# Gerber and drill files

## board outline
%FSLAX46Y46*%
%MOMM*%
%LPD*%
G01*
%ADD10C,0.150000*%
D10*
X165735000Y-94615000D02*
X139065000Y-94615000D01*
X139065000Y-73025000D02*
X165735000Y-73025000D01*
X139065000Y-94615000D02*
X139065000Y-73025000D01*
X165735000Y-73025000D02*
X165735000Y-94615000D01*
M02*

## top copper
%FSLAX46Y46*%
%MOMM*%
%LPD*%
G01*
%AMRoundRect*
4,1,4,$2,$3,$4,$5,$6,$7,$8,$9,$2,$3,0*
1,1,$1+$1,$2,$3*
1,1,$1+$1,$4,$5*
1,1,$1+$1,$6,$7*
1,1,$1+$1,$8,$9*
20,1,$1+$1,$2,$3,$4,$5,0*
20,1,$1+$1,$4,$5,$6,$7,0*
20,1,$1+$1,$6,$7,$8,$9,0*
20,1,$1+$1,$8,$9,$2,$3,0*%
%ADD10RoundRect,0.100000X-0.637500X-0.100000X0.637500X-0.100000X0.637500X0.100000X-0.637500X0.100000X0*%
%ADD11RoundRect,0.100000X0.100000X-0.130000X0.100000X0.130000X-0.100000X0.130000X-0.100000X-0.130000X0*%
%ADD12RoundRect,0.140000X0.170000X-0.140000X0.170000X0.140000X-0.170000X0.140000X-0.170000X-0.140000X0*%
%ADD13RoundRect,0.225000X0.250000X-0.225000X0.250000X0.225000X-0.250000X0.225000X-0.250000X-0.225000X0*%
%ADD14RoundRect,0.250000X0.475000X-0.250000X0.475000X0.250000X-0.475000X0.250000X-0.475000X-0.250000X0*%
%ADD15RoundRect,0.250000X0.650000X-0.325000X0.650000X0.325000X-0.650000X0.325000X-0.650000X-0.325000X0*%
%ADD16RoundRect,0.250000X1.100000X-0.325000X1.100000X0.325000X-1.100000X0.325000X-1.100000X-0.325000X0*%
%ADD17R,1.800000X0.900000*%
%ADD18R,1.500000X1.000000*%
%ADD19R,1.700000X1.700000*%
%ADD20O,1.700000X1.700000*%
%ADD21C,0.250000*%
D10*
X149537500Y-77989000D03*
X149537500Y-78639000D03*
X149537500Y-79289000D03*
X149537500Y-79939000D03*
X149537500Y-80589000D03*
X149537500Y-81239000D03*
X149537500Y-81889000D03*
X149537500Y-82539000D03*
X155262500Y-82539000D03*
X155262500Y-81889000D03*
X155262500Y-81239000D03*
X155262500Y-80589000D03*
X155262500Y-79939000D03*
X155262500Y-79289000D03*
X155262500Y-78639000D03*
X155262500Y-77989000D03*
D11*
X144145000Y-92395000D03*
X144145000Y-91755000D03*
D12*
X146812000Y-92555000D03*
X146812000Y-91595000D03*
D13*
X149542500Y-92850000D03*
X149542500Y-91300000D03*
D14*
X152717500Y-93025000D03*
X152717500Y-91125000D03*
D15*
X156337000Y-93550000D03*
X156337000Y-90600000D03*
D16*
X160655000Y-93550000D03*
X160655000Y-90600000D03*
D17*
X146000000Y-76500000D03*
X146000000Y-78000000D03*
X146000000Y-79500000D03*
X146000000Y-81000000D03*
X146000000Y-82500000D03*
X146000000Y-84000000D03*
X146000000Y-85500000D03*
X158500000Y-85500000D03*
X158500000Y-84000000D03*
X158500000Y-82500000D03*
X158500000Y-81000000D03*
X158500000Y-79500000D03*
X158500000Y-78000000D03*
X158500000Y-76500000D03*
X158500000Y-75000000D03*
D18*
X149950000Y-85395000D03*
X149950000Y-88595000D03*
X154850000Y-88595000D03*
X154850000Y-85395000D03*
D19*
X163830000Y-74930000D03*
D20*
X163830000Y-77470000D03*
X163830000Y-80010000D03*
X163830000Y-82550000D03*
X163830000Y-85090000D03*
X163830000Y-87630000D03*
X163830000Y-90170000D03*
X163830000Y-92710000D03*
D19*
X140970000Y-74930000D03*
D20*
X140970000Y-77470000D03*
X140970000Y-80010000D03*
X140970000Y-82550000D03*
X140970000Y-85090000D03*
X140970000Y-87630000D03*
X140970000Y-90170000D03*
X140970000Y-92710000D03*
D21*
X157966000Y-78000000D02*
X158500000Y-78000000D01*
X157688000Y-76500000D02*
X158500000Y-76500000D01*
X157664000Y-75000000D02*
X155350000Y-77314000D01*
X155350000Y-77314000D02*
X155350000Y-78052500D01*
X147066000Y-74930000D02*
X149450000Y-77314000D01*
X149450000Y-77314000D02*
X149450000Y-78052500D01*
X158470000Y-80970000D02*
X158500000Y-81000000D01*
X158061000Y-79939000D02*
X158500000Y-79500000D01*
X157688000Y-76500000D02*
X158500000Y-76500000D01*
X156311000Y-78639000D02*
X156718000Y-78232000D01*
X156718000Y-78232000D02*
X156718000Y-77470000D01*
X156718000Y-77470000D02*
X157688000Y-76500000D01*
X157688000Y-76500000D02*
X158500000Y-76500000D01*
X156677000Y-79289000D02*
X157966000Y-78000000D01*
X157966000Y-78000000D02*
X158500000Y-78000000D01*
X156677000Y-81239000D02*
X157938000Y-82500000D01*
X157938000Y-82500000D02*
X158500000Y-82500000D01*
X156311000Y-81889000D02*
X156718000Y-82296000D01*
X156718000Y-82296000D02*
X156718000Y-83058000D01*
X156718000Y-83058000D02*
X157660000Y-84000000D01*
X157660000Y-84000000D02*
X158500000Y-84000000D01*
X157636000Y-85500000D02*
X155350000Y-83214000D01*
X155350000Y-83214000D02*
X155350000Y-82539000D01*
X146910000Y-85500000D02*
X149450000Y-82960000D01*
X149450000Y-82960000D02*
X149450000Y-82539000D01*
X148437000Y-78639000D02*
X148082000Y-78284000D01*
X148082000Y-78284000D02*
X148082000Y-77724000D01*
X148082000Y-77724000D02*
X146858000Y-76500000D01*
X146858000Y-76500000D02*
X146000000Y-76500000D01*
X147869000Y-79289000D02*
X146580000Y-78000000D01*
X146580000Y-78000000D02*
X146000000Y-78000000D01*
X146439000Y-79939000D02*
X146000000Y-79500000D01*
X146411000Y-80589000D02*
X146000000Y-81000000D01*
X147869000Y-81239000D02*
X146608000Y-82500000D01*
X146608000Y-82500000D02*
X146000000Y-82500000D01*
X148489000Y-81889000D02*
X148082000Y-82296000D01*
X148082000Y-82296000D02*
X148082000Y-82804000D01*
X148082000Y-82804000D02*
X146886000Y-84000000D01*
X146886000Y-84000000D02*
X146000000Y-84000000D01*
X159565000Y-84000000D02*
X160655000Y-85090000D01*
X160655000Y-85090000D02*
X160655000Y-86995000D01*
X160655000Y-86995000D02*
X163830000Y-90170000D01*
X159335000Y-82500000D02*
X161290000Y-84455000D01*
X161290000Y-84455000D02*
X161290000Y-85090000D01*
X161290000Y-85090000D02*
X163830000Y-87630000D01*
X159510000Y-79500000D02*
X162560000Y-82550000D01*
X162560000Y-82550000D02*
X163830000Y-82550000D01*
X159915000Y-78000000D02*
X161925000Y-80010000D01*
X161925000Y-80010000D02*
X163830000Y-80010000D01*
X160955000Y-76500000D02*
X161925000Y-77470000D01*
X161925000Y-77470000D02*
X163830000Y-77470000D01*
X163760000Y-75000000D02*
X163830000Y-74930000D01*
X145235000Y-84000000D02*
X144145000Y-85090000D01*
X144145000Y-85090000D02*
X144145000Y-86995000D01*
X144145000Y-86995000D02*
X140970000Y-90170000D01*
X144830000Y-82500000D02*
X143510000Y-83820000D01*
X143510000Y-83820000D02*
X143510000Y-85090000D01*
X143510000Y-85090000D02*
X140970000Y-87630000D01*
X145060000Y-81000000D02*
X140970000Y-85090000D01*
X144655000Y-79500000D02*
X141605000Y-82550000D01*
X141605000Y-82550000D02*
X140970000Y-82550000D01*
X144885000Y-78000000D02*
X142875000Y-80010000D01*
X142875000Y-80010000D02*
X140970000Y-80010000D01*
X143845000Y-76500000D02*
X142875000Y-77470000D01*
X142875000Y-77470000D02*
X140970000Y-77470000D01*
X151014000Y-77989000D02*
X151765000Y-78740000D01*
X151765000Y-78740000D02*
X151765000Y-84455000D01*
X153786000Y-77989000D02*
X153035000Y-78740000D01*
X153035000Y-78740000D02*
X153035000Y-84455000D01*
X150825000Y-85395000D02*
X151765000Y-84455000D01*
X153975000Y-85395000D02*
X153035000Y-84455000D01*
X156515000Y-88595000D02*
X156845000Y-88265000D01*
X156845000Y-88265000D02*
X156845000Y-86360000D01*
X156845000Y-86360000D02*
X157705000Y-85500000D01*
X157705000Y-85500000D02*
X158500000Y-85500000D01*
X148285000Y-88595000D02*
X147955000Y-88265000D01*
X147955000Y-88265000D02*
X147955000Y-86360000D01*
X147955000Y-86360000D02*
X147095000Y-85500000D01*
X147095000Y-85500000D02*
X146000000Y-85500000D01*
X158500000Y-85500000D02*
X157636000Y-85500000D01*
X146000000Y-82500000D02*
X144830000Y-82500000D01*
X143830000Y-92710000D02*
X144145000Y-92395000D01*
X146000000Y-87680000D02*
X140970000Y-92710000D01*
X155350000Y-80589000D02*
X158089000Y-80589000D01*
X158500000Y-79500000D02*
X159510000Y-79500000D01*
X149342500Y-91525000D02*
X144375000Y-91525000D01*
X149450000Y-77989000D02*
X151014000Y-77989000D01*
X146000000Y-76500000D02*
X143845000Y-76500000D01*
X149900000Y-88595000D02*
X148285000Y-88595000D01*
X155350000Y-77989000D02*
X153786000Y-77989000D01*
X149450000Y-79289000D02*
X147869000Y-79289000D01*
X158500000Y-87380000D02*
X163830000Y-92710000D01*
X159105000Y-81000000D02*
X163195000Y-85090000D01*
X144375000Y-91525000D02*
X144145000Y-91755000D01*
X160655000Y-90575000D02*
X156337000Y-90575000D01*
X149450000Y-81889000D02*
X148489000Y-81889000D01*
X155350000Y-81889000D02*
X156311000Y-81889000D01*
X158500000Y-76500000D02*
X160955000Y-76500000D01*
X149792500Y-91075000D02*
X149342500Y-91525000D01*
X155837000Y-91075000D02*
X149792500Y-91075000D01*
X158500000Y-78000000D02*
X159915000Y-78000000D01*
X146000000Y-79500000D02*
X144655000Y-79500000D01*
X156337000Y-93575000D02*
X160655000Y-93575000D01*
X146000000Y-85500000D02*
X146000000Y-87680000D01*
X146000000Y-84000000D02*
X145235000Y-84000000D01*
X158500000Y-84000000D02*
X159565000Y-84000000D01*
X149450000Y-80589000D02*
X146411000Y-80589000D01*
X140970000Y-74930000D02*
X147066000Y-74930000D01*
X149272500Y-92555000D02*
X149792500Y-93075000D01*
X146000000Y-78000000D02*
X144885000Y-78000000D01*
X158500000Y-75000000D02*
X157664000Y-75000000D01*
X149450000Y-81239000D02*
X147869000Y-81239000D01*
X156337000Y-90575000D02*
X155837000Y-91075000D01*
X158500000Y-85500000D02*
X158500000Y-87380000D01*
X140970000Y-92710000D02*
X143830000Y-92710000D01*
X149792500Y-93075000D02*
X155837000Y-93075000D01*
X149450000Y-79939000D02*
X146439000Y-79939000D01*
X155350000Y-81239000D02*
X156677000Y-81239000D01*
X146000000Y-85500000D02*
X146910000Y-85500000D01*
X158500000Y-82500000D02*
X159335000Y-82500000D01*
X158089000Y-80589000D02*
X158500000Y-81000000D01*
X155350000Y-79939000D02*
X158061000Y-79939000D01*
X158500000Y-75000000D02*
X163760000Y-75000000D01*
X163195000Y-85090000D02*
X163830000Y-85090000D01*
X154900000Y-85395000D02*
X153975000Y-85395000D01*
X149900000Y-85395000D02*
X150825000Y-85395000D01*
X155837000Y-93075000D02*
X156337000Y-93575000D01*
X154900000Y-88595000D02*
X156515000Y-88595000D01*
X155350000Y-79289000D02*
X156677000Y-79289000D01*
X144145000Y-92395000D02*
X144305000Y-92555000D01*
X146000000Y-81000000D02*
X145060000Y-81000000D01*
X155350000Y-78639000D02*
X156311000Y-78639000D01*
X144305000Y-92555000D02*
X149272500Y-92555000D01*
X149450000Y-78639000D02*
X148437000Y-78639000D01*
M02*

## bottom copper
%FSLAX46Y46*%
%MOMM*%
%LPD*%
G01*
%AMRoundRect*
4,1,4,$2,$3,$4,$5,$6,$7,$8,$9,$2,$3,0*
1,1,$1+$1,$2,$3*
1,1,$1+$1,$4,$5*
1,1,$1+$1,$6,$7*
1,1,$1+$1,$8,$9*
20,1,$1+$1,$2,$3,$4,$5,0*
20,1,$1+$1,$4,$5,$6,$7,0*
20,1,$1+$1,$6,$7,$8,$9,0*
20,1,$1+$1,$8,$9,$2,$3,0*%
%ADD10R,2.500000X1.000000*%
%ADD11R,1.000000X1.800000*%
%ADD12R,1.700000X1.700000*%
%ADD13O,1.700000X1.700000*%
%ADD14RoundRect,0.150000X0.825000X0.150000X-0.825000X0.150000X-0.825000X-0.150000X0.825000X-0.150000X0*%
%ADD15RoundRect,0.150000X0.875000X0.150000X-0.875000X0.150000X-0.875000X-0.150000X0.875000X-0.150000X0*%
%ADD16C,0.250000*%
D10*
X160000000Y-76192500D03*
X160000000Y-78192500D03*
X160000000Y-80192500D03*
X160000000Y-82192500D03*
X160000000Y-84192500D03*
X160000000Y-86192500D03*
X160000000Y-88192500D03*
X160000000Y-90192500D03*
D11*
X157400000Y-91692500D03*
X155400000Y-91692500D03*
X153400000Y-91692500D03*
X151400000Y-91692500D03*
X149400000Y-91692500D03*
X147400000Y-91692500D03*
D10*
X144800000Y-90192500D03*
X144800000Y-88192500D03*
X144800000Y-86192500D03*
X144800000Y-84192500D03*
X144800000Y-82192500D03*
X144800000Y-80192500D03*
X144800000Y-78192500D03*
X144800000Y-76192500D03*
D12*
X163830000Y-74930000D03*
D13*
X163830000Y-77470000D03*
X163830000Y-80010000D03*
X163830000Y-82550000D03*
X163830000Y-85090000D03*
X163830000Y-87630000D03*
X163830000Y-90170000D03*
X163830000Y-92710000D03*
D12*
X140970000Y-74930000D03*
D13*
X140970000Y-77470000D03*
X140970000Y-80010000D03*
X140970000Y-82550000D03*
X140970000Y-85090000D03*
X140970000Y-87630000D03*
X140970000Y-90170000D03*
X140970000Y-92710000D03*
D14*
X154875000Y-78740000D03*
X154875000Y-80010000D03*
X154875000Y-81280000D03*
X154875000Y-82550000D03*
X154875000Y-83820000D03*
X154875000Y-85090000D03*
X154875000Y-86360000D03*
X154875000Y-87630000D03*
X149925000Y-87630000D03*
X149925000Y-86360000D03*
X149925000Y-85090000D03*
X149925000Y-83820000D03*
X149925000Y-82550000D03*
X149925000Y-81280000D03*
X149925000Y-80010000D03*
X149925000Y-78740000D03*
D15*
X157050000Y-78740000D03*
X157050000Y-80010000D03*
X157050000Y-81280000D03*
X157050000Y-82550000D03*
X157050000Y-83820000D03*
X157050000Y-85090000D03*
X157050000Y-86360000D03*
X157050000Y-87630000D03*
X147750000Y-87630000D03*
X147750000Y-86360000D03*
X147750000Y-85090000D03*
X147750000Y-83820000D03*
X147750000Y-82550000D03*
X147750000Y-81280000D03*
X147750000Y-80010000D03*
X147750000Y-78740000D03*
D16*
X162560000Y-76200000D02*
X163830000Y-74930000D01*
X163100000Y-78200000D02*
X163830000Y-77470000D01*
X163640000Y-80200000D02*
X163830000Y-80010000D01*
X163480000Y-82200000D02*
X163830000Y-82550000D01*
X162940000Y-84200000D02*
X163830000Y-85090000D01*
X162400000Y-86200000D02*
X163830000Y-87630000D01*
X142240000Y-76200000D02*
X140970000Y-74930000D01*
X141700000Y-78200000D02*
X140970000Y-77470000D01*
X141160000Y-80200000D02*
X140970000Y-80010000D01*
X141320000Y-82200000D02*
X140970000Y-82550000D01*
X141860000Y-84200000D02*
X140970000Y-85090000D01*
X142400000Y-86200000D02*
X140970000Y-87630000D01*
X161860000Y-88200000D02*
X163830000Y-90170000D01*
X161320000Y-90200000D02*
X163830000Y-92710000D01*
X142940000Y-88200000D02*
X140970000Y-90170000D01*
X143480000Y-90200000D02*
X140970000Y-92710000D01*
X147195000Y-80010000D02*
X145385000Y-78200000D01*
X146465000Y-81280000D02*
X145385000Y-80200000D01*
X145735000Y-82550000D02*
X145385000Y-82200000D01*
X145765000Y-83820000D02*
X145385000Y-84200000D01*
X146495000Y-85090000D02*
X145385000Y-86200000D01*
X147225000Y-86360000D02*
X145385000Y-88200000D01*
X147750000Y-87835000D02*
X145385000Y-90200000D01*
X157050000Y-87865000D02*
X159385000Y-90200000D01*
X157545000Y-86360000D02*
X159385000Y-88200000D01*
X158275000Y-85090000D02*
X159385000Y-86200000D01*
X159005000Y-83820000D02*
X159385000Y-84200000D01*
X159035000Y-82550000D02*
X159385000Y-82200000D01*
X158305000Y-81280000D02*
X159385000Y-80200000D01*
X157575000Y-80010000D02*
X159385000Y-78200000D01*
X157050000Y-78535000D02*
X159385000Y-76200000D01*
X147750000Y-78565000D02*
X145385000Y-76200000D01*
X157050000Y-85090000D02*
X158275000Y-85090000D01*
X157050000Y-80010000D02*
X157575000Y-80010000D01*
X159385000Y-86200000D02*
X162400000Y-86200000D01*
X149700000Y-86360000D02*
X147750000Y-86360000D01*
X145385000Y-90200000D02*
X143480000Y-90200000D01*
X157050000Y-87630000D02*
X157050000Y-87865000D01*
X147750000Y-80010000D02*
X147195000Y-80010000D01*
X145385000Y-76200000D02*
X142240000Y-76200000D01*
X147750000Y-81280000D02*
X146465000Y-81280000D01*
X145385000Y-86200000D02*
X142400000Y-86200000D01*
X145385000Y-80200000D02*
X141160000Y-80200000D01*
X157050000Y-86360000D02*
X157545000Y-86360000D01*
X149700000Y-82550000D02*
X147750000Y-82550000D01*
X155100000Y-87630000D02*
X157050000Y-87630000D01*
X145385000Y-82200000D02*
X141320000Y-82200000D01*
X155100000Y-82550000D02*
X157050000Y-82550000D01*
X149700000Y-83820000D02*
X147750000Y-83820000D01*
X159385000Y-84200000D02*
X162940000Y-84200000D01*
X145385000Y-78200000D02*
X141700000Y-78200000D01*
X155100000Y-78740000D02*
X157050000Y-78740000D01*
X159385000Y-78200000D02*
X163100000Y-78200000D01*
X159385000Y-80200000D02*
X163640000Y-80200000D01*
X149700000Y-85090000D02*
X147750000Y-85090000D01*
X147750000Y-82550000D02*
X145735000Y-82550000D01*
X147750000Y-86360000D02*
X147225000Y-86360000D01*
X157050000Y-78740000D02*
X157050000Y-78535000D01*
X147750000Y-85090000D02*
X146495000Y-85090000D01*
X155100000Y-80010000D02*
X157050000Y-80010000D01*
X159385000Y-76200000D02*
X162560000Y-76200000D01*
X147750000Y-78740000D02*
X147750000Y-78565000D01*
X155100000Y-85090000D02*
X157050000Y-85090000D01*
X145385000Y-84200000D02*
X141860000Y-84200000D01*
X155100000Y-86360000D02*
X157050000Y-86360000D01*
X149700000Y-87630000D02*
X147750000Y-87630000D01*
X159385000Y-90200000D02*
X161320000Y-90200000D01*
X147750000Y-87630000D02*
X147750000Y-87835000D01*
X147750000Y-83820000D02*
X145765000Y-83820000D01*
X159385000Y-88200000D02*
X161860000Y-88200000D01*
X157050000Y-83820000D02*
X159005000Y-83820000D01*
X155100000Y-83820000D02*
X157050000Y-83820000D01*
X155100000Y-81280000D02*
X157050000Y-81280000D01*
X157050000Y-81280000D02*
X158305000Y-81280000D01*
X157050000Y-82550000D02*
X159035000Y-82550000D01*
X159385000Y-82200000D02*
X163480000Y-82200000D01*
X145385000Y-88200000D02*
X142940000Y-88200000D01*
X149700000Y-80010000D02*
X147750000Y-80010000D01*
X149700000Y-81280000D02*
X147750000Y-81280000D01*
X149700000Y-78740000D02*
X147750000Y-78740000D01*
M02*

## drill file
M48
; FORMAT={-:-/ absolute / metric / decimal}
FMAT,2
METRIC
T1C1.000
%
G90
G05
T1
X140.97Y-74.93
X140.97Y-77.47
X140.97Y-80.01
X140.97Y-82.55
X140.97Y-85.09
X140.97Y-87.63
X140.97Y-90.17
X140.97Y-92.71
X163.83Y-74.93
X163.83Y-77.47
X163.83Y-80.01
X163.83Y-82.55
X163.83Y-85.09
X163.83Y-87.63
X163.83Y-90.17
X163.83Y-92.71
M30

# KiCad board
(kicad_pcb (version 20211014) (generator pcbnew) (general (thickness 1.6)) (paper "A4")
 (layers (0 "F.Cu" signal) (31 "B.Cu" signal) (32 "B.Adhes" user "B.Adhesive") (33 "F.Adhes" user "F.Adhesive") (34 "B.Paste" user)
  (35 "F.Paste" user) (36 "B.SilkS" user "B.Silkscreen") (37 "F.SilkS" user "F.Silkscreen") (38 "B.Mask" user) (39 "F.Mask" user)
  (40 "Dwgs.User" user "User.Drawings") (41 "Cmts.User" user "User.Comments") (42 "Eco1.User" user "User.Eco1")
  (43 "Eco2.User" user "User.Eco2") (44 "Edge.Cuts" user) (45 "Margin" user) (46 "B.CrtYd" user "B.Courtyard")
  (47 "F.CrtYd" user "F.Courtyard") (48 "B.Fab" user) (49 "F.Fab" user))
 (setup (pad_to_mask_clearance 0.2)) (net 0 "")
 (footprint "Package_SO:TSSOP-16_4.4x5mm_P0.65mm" (layer "F.Cu") (at 152.4 80.264)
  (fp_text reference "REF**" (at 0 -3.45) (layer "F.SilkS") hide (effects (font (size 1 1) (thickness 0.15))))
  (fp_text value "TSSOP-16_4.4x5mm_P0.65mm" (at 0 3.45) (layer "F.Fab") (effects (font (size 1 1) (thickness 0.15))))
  (pad "1" smd roundrect (at -2.8625 -2.275) (size 1.475 0.4) (layers "F.Cu" "F.Paste" "F.Mask") (roundrect_rratio 0.25))
  (pad "2" smd roundrect (at -2.8625 -1.625) (size 1.475 0.4) (layers "F.Cu" "F.Paste" "F.Mask") (roundrect_rratio 0.25))
  (pad "3" smd roundrect (at -2.8625 -0.975) (size 1.475 0.4) (layers "F.Cu" "F.Paste" "F.Mask") (roundrect_rratio 0.25))
  (pad "4" smd roundrect (at -2.8625 -0.325) (size 1.475 0.4) (layers "F.Cu" "F.Paste" "F.Mask") (roundrect_rratio 0.25))
  (pad "5" smd roundrect (at -2.8625 0.325) (size 1.475 0.4) (layers "F.Cu" "F.Paste" "F.Mask") (roundrect_rratio 0.25))
  (pad "6" smd roundrect (at -2.8625 0.975) (size 1.475 0.4) (layers "F.Cu" "F.Paste" "F.Mask") (roundrect_rratio 0.25))
  (pad "7" smd roundrect (at -2.8625 1.625) (size 1.475 0.4) (layers "F.Cu" "F.Paste" "F.Mask") (roundrect_rratio 0.25))
  (pad "8" smd roundrect (at -2.8625 2.275) (size 1.475 0.4) (layers "F.Cu" "F.Paste" "F.Mask") (roundrect_rratio 0.25))
  (pad "9" smd roundrect (at 2.8625 2.275) (size 1.475 0.4) (layers "F.Cu" "F.Paste" "F.Mask") (roundrect_rratio 0.25))
  (pad "10" smd roundrect (at 2.8625 1.625) (size 1.475 0.4) (layers "F.Cu" "F.Paste" "F.Mask") (roundrect_rratio 0.25))
  (pad "11" smd roundrect (at 2.8625 0.975) (size 1.475 0.4) (layers "F.Cu" "F.Paste" "F.Mask") (roundrect_rratio 0.25))
  (pad "12" smd roundrect (at 2.8625 0.325) (size 1.475 0.4) (layers "F.Cu" "F.Paste" "F.Mask") (roundrect_rratio 0.25))
  (pad "13" smd roundrect (at 2.8625 -0.325) (size 1.475 0.4) (layers "F.Cu" "F.Paste" "F.Mask") (roundrect_rratio 0.25))
  (pad "14" smd roundrect (at 2.8625 -0.975) (size 1.475 0.4) (layers "F.Cu" "F.Paste" "F.Mask") (roundrect_rratio 0.25))
  (pad "15" smd roundrect (at 2.8625 -1.625) (size 1.475 0.4) (layers "F.Cu" "F.Paste" "F.Mask") (roundrect_rratio 0.25))
  (pad "16" smd roundrect (at 2.8625 -2.275) (size 1.475 0.4) (layers "F.Cu" "F.Paste" "F.Mask") (roundrect_rratio 0.25)))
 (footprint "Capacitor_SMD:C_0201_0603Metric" (layer "F.Cu") (at 144.145 92.075 90)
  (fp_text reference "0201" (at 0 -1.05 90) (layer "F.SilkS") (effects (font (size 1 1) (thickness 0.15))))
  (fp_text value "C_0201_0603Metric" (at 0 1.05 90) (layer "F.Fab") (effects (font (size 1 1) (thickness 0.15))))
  (pad "" smd roundrect (at -0.345 0 90) (size 0.318 0.36) (layers "F.Paste") (roundrect_rratio 0.25))
  (pad "" smd roundrect (at 0.345 0 90) (size 0.318 0.36) (layers "F.Paste") (roundrect_rratio 0.25))
  (pad "1" smd roundrect (at -0.32 0 90) (size 0.46 0.4) (layers "F.Cu" "F.Mask") (roundrect_rratio 0.25))
  (pad "2" smd roundrect (at 0.32 0 90) (size 0.46 0.4) (layers "F.Cu" "F.Mask") (roundrect_rratio 0.25)))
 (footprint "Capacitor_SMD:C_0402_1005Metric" (layer "F.Cu") (at 146.812 92.075 90)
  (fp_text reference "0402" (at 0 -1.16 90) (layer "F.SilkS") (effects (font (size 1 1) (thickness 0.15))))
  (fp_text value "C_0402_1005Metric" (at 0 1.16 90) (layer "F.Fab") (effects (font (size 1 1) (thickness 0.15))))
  (pad "1" smd roundrect (at -0.48 0 90) (size 0.56 0.62) (layers "F.Cu" "F.Paste" "F.Mask") (roundrect_rratio 0.25))
  (pad "2" smd roundrect (at 0.48 0 90) (size 0.56 0.62) (layers "F.Cu" "F.Paste" "F.Mask") (roundrect_rratio 0.25)))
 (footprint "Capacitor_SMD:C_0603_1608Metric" (layer "F.Cu") (at 149.5425 92.075 90)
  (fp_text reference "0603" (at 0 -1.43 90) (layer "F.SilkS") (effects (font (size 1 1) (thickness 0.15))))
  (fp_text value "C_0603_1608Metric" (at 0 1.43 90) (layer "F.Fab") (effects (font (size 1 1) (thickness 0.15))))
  (pad "1" smd roundrect (at -0.775 0 90) (size 0.9 0.95) (layers "F.Cu" "F.Paste" "F.Mask") (roundrect_rratio 0.25))
  (pad "2" smd roundrect (at 0.775 0 90) (size 0.9 0.95) (layers "F.Cu" "F.Paste" "F.Mask") (roundrect_rratio 0.25)))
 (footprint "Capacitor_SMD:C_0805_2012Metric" (layer "F.Cu") (at 152.7175 92.075 90)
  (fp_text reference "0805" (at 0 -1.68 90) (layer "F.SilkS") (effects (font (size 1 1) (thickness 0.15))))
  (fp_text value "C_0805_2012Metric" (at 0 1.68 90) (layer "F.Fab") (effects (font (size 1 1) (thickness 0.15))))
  (pad "1" smd roundrect (at -0.95 0 90) (size 1 1.45) (layers "F.Cu" "F.Paste" "F.Mask") (roundrect_rratio 0.25))
  (pad "2" smd roundrect (at 0.95 0 90) (size 1 1.45) (layers "F.Cu" "F.Paste" "F.Mask") (roundrect_rratio 0.25)))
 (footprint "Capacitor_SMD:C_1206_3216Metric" (layer "F.Cu") (at 156.337 92.075 90)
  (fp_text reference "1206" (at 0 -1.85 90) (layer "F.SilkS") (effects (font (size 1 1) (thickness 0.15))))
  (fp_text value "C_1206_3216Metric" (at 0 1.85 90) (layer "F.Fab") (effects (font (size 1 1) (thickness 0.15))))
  (pad "1" smd roundrect (at -1.475 0 90) (size 1.15 1.8) (layers "F.Cu" "F.Paste" "F.Mask") (roundrect_rratio 0.217391))
  (pad "2" smd roundrect (at 1.475 0 90) (size 1.15 1.8) (layers "F.Cu" "F.Paste" "F.Mask") (roundrect_rratio 0.217391)))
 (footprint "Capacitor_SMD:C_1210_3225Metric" (layer "F.Cu") (at 160.655 92.075 90)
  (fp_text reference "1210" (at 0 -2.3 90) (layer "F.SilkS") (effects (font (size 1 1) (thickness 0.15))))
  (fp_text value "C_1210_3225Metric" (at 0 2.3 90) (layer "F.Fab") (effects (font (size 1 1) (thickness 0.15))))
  (pad "1" smd roundrect (at -1.475 0 90) (size 1.15 2.7) (layers "F.Cu" "F.Paste" "F.Mask") (roundrect_rratio 0.217391))
  (pad "2" smd roundrect (at 1.475 0 90) (size 1.15 2.7) (layers "F.Cu" "F.Paste" "F.Mask") (roundrect_rratio 0.217391)))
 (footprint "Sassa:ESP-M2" (layer "F.Cu") (at 146 76.5)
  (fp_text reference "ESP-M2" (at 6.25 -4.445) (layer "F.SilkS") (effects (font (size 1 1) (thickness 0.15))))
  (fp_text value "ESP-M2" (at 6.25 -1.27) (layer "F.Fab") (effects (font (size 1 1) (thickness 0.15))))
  (pad "1" smd rect (at 0 0) (size 1.8 0.9) (layers "F.Cu" "F.Paste" "F.Mask"))
  (pad "2" smd rect (at 0 1.5) (size 1.8 0.9) (layers "F.Cu" "F.Paste" "F.Mask"))
  (pad "3" smd rect (at 0 3) (size 1.8 0.9) (layers "F.Cu" "F.Paste" "F.Mask"))
  (pad "4" smd rect (at 0 4.5) (size 1.8 0.9) (layers "F.Cu" "F.Paste" "F.Mask"))
  (pad "5" smd rect (at 0 6) (size 1.8 0.9) (layers "F.Cu" "F.Paste" "F.Mask"))
  (pad "6" smd rect (at 0 7.5) (size 1.8 0.9) (layers "F.Cu" "F.Paste" "F.Mask"))
  (pad "7" smd rect (at 0 9) (size 1.8 0.9) (layers "F.Cu" "F.Paste" "F.Mask"))
  (pad "8" smd rect (at 12.5 9) (size 1.8 0.9) (layers "F.Cu" "F.Paste" "F.Mask"))
  (pad "9" smd rect (at 12.5 7.5) (size 1.8 0.9) (layers "F.Cu" "F.Paste" "F.Mask"))
  (pad "10" smd rect (at 12.5 6) (size 1.8 0.9) (layers "F.Cu" "F.Paste" "F.Mask"))
  (pad "11" smd rect (at 12.5 4.5) (size 1.8 0.9) (layers "F.Cu" "F.Paste" "F.Mask"))
  (pad "12" smd rect (at 12.5 3) (size 1.8 0.9) (layers "F.Cu" "F.Paste" "F.Mask"))
  (pad "13" smd rect (at 12.5 1.5) (size 1.8 0.9) (layers "F.Cu" "F.Paste" "F.Mask"))
  (pad "14" smd rect (at 12.5 0) (size 1.8 0.9) (layers "F.Cu" "F.Paste" "F.Mask"))
  (pad "15" smd rect (at 12.5 -1.5) (size 1.8 0.9) (layers "F.Cu" "F.Paste" "F.Mask")))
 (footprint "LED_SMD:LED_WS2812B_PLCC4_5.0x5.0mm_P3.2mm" (layer "F.Cu") (at 152.4 86.995)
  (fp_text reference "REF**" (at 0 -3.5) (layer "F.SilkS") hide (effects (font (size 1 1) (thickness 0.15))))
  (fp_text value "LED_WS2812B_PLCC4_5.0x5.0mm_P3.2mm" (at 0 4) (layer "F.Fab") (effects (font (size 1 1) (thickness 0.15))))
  (pad "1" smd rect (at -2.45 -1.6) (size 1.5 1) (layers "F.Cu" "F.Paste" "F.Mask"))
  (pad "2" smd rect (at -2.45 1.6) (size 1.5 1) (layers "F.Cu" "F.Paste" "F.Mask"))
  (pad "3" smd rect (at 2.45 1.6) (size 1.5 1) (layers "F.Cu" "F.Paste" "F.Mask"))
  (pad "4" smd rect (at 2.45 -1.6) (size 1.5 1) (layers "F.Cu" "F.Paste" "F.Mask")))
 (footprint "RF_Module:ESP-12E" (layer "B.Cu") (at 152.4 79.6925 180)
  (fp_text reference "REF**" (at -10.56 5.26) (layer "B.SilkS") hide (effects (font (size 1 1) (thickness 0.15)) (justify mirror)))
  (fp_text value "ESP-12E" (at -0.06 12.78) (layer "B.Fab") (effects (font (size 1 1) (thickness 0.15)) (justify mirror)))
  (pad "1" smd rect (at -7.6 3.5 180) (size 2.5 1) (layers "B.Cu" "B.Paste" "B.Mask"))
  (pad "2" smd rect (at -7.6 1.5 180) (size 2.5 1) (layers "B.Cu" "B.Paste" "B.Mask"))
  (pad "3" smd rect (at -7.6 -0.5 180) (size 2.5 1) (layers "B.Cu" "B.Paste" "B.Mask"))
  (pad "4" smd rect (at -7.6 -2.5 180) (size 2.5 1) (layers "B.Cu" "B.Paste" "B.Mask"))
  (pad "5" smd rect (at -7.6 -4.5 180) (size 2.5 1) (layers "B.Cu" "B.Paste" "B.Mask"))
  (pad "6" smd rect (at -7.6 -6.5 180) (size 2.5 1) (layers "B.Cu" "B.Paste" "B.Mask"))
  (pad "7" smd rect (at -7.6 -8.5 180) (size 2.5 1) (layers "B.Cu" "B.Paste" "B.Mask"))
  (pad "8" smd rect (at -7.6 -10.5 180) (size 2.5 1) (layers "B.Cu" "B.Paste" "B.Mask"))
  (pad "9" smd rect (at -5 -12 180) (size 1 1.8) (layers "B.Cu" "B.Paste" "B.Mask"))
  (pad "10" smd rect (at -3 -12 180) (size 1 1.8) (layers "B.Cu" "B.Paste" "B.Mask"))
  (pad "11" smd rect (at -1 -12 180) (size 1 1.8) (layers "B.Cu" "B.Paste" "B.Mask"))
  (pad "12" smd rect (at 1 -12 180) (size 1 1.8) (layers "B.Cu" "B.Paste" "B.Mask"))
  (pad "13" smd rect (at 3 -12 180) (size 1 1.8) (layers "B.Cu" "B.Paste" "B.Mask"))
  (pad "14" smd rect (at 5 -12 180) (size 1 1.8) (layers "B.Cu" "B.Paste" "B.Mask"))
  (pad "15" smd rect (at 7.6 -10.5 180) (size 2.5 1) (layers "B.Cu" "B.Paste" "B.Mask"))
  (pad "16" smd rect (at 7.6 -8.5 180) (size 2.5 1) (layers "B.Cu" "B.Paste" "B.Mask"))
  (pad "17" smd rect (at 7.6 -6.5 180) (size 2.5 1) (layers "B.Cu" "B.Paste" "B.Mask"))
  (pad "18" smd rect (at 7.6 -4.5 180) (size 2.5 1) (layers "B.Cu" "B.Paste" "B.Mask"))
  (pad "19" smd rect (at 7.6 -2.5 180) (size 2.5 1) (layers "B.Cu" "B.Paste" "B.Mask"))
  (pad "20" smd rect (at 7.6 -0.5 180) (size 2.5 1) (layers "B.Cu" "B.Paste" "B.Mask"))
  (pad "21" smd rect (at 7.6 1.5 180) (size 2.5 1) (layers "B.Cu" "B.Paste" "B.Mask"))
  (pad "22" smd rect (at 7.6 3.5 180) (size 2.5 1) (layers "B.Cu" "B.Paste" "B.Mask"))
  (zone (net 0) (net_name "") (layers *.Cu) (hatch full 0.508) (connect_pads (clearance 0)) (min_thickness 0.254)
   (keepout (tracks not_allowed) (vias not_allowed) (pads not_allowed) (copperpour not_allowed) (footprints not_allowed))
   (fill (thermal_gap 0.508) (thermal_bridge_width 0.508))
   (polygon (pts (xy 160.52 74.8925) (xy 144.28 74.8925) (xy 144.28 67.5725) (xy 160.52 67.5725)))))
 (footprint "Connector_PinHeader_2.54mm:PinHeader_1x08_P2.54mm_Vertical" (layer "B.Cu") (at 163.83 74.93 180)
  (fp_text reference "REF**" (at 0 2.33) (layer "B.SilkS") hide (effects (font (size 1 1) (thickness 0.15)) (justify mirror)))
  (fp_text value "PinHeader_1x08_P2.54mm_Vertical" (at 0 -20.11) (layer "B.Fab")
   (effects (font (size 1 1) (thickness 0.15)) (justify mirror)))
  (pad "1" thru_hole rect (at 0 0 180) (size 1.7 1.7) (drill 1) (layers *.Cu *.Mask))
  (pad "2" thru_hole oval (at 0 -2.54 180) (size 1.7 1.7) (drill 1) (layers *.Cu *.Mask))
  (pad "3" thru_hole oval (at 0 -5.08 180) (size 1.7 1.7) (drill 1) (layers *.Cu *.Mask))
  (pad "4" thru_hole oval (at 0 -7.62 180) (size 1.7 1.7) (drill 1) (layers *.Cu *.Mask))
  (pad "5" thru_hole oval (at 0 -10.16 180) (size 1.7 1.7) (drill 1) (layers *.Cu *.Mask))
  (pad "6" thru_hole oval (at 0 -12.7 180) (size 1.7 1.7) (drill 1) (layers *.Cu *.Mask))
  (pad "7" thru_hole oval (at 0 -15.24 180) (size 1.7 1.7) (drill 1) (layers *.Cu *.Mask))
  (pad "8" thru_hole oval (at 0 -17.78 180) (size 1.7 1.7) (drill 1) (layers *.Cu *.Mask)))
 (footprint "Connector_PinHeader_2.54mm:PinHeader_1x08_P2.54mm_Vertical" (layer "B.Cu") (at 140.97 74.93 180)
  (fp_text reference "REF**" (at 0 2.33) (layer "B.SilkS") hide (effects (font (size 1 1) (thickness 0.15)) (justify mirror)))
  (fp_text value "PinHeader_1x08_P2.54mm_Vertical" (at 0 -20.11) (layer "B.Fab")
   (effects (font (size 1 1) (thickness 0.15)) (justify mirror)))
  (pad "1" thru_hole rect (at 0 0 180) (size 1.7 1.7) (drill 1) (layers *.Cu *.Mask))
  (pad "2" thru_hole oval (at 0 -2.54 180) (size 1.7 1.7) (drill 1) (layers *.Cu *.Mask))
  (pad "3" thru_hole oval (at 0 -5.08 180) (size 1.7 1.7) (drill 1) (layers *.Cu *.Mask))
  (pad "4" thru_hole oval (at 0 -7.62 180) (size 1.7 1.7) (drill 1) (layers *.Cu *.Mask))
  (pad "5" thru_hole oval (at 0 -10.16 180) (size 1.7 1.7) (drill 1) (layers *.Cu *.Mask))
  (pad "6" thru_hole oval (at 0 -12.7 180) (size 1.7 1.7) (drill 1) (layers *.Cu *.Mask))
  (pad "7" thru_hole oval (at 0 -15.24 180) (size 1.7 1.7) (drill 1) (layers *.Cu *.Mask))
  (pad "8" thru_hole oval (at 0 -17.78 180) (size 1.7 1.7) (drill 1) (layers *.Cu *.Mask)))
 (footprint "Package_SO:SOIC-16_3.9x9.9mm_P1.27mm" (layer "B.Cu") (at 152.4 83.185 180)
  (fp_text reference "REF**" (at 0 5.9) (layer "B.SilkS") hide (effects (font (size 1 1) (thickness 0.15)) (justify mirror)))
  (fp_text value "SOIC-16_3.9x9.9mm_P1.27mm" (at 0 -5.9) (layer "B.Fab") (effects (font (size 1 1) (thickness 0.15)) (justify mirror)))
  (pad "1" smd roundrect (at -2.475 4.445 180) (size 1.95 0.6) (layers "B.Cu" "B.Paste" "B.Mask") (roundrect_rratio 0.25))
  (pad "2" smd roundrect (at -2.475 3.175 180) (size 1.95 0.6) (layers "B.Cu" "B.Paste" "B.Mask") (roundrect_rratio 0.25))
  (pad "3" smd roundrect (at -2.475 1.905 180) (size 1.95 0.6) (layers "B.Cu" "B.Paste" "B.Mask") (roundrect_rratio 0.25))
  (pad "4" smd roundrect (at -2.475 0.635 180) (size 1.95 0.6) (layers "B.Cu" "B.Paste" "B.Mask") (roundrect_rratio 0.25))
  (pad "5" smd roundrect (at -2.475 -0.635 180) (size 1.95 0.6) (layers "B.Cu" "B.Paste" "B.Mask") (roundrect_rratio 0.25))
  (pad "6" smd roundrect (at -2.475 -1.905 180) (size 1.95 0.6) (layers "B.Cu" "B.Paste" "B.Mask") (roundrect_rratio 0.25))
  (pad "7" smd roundrect (at -2.475 -3.175 180) (size 1.95 0.6) (layers "B.Cu" "B.Paste" "B.Mask") (roundrect_rratio 0.25))
  (pad "8" smd roundrect (at -2.475 -4.445 180) (size 1.95 0.6) (layers "B.Cu" "B.Paste" "B.Mask") (roundrect_rratio 0.25))
  (pad "9" smd roundrect (at 2.475 -4.445 180) (size 1.95 0.6) (layers "B.Cu" "B.Paste" "B.Mask") (roundrect_rratio 0.25))
  (pad "10" smd roundrect (at 2.475 -3.175 180) (size 1.95 0.6) (layers "B.Cu" "B.Paste" "B.Mask") (roundrect_rratio 0.25))
  (pad "11" smd roundrect (at 2.475 -1.905 180) (size 1.95 0.6) (layers "B.Cu" "B.Paste" "B.Mask") (roundrect_rratio 0.25))
  (pad "12" smd roundrect (at 2.475 -0.635 180) (size 1.95 0.6) (layers "B.Cu" "B.Paste" "B.Mask") (roundrect_rratio 0.25))
  (pad "13" smd roundrect (at 2.475 0.635 180) (size 1.95 0.6) (layers "B.Cu" "B.Paste" "B.Mask") (roundrect_rratio 0.25))
  (pad "14" smd roundrect (at 2.475 1.905 180) (size 1.95 0.6) (layers "B.Cu" "B.Paste" "B.Mask") (roundrect_rratio 0.25))
  (pad "15" smd roundrect (at 2.475 3.175 180) (size 1.95 0.6) (layers "B.Cu" "B.Paste" "B.Mask") (roundrect_rratio 0.25))
  (pad "16" smd roundrect (at 2.475 4.445 180) (size 1.95 0.6) (layers "B.Cu" "B.Paste" "B.Mask") (roundrect_rratio 0.25)))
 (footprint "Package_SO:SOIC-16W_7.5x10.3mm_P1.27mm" (layer "B.Cu") (at 152.4 83.185 180)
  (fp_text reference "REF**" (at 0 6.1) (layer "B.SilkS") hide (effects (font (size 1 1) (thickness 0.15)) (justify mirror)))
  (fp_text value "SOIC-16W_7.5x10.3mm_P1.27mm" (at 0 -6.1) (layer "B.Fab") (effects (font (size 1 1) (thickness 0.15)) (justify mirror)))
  (pad "1" smd roundrect (at -4.65 4.445 180) (size 2.05 0.6) (layers "B.Cu" "B.Paste" "B.Mask") (roundrect_rratio 0.25))
  (pad "2" smd roundrect (at -4.65 3.175 180) (size 2.05 0.6) (layers "B.Cu" "B.Paste" "B.Mask") (roundrect_rratio 0.25))
  (pad "3" smd roundrect (at -4.65 1.905 180) (size 2.05 0.6) (layers "B.Cu" "B.Paste" "B.Mask") (roundrect_rratio 0.25))
  (pad "4" smd roundrect (at -4.65 0.635 180) (size 2.05 0.6) (layers "B.Cu" "B.Paste" "B.Mask") (roundrect_rratio 0.25))
  (pad "5" smd roundrect (at -4.65 -0.635 180) (size 2.05 0.6) (layers "B.Cu" "B.Paste" "B.Mask") (roundrect_rratio 0.25))
  (pad "6" smd roundrect (at -4.65 -1.905 180) (size 2.05 0.6) (layers "B.Cu" "B.Paste" "B.Mask") (roundrect_rratio 0.25))
  (pad "7" smd roundrect (at -4.65 -3.175 180) (size 2.05 0.6) (layers "B.Cu" "B.Paste" "B.Mask") (roundrect_rratio 0.25))
  (pad "8" smd roundrect (at -4.65 -4.445 180) (size 2.05 0.6) (layers "B.Cu" "B.Paste" "B.Mask") (roundrect_rratio 0.25))
  (pad "9" smd roundrect (at 4.65 -4.445 180) (size 2.05 0.6) (layers "B.Cu" "B.Paste" "B.Mask") (roundrect_rratio 0.25))
  (pad "10" smd roundrect (at 4.65 -3.175 180) (size 2.05 0.6) (layers "B.Cu" "B.Paste" "B.Mask") (roundrect_rratio 0.25))
  (pad "11" smd roundrect (at 4.65 -1.905 180) (size 2.05 0.6) (layers "B.Cu" "B.Paste" "B.Mask") (roundrect_rratio 0.25))
  (pad "12" smd roundrect (at 4.65 -0.635 180) (size 2.05 0.6) (layers "B.Cu" "B.Paste" "B.Mask") (roundrect_rratio 0.25))
  (pad "13" smd roundrect (at 4.65 0.635 180) (size 2.05 0.6) (layers "B.Cu" "B.Paste" "B.Mask") (roundrect_rratio 0.25))
  (pad "14" smd roundrect (at 4.65 1.905 180) (size 2.05 0.6) (layers "B.Cu" "B.Paste" "B.Mask") (roundrect_rratio 0.25))
  (pad "15" smd roundrect (at 4.65 3.175 180) (size 2.05 0.6) (layers "B.Cu" "B.Paste" "B.Mask") (roundrect_rratio 0.25))
  (pad "16" smd roundrect (at 4.65 4.445 180) (size 2.05 0.6) (layers "B.Cu" "B.Paste" "B.Mask") (roundrect_rratio 0.25)))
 (gr_line (start 165.735 94.615) (end 139.065 94.615) (layer "Edge.Cuts") (width 0.15))
 (gr_line (start 139.065 73.025) (end 165.735 73.025) (layer "Edge.Cuts") (width 0.15))
 (gr_line (start 139.065 94.615) (end 139.065 73.025) (layer "Edge.Cuts") (width 0.15))
 (gr_line (start 165.735 73.025) (end 165.735 94.615) (layer "Edge.Cuts") (width 0.15))
 (segment (start 157.966 78) (end 158.5 78) (width 0.25) (layer "F.Cu") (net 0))
 (segment (start 157.688 76.5) (end 158.5 76.5) (width 0.25) (layer "F.Cu") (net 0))
 (segment (start 157.664 75) (end 155.35 77.314) (width 0.25) (layer "F.Cu") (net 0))
 (segment (start 155.35 77.314) (end 155.35 78.0525) (width 0.25) (layer "F.Cu") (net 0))
 (segment (start 147.066 74.93) (end 149.45 77.314) (width 0.25) (layer "F.Cu") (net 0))
 (segment (start 149.45 77.314) (end 149.45 78.0525) (width 0.25) (layer "F.Cu") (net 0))
 (segment (start 158.47 80.97) (end 158.5 81) (width 0.25) (layer "F.Cu") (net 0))
 (segment (start 158.061 79.939) (end 158.5 79.5) (width 0.25) (layer "F.Cu") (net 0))
 (segment (start 157.688 76.5) (end 158.5 76.5) (width 0.25) (layer "F.Cu") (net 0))
 (segment (start 156.311 78.639) (end 156.718 78.232) (width 0.25) (layer "F.Cu") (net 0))
 (segment (start 156.718 78.232) (end 156.718 77.47) (width 0.25) (layer "F.Cu") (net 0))
 (segment (start 156.718 77.47) (end 157.688 76.5) (width 0.25) (layer "F.Cu") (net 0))
 (segment (start 157.688 76.5) (end 158.5 76.5) (width 0.25) (layer "F.Cu") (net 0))
 (segment (start 156.677 79.289) (end 157.966 78) (width 0.25) (layer "F.Cu") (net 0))
 (segment (start 157.966 78) (end 158.5 78) (width 0.25) (layer "F.Cu") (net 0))
 (segment (start 156.677 81.239) (end 157.938 82.5) (width 0.25) (layer "F.Cu") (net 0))
 (segment (start 157.938 82.5) (end 158.5 82.5) (width 0.25) (layer "F.Cu") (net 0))
 (segment (start 156.311 81.889) (end 156.718 82.296) (width 0.25) (layer "F.Cu") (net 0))
 (segment (start 156.718 82.296) (end 156.718 83.058) (width 0.25) (layer "F.Cu") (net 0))
 (segment (start 156.718 83.058) (end 157.66 84) (width 0.25) (layer "F.Cu") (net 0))
 (segment (start 157.66 84) (end 158.5 84) (width 0.25) (layer "F.Cu") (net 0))
 (segment (start 157.636 85.5) (end 155.35 83.214) (width 0.25) (layer "F.Cu") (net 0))
 (segment (start 155.35 83.214) (end 155.35 82.539) (width 0.25) (layer "F.Cu") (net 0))
 (segment (start 146.91 85.5) (end 149.45 82.96) (width 0.25) (layer "F.Cu") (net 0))
 (segment (start 149.45 82.96) (end 149.45 82.539) (width 0.25) (layer "F.Cu") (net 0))
 (segment (start 148.437 78.639) (end 148.082 78.284) (width 0.25) (layer "F.Cu") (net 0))
 (segment (start 148.082 78.284) (end 148.082 77.724) (width 0.25) (layer "F.Cu") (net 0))
 (segment (start 148.082 77.724) (end 146.858 76.5) (width 0.25) (layer "F.Cu") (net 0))
 (segment (start 146.858 76.5) (end 146 76.5) (width 0.25) (layer "F.Cu") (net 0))
 (segment (start 147.869 79.289) (end 146.58 78) (width 0.25) (layer "F.Cu") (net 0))
 (segment (start 146.58 78) (end 146 78) (width 0.25) (layer "F.Cu") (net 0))
 (segment (start 146.439 79.939) (end 146 79.5) (width 0.25) (layer "F.Cu") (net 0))
 (segment (start 146.411 80.589) (end 146 81) (width 0.25) (layer "F.Cu") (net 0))
 (segment (start 147.869 81.239) (end 146.608 82.5) (width 0.25) (layer "F.Cu") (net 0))
 (segment (start 146.608 82.5) (end 146 82.5) (width 0.25) (layer "F.Cu") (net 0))
 (segment (start 148.489 81.889) (end 148.082 82.296) (width 0.25) (layer "F.Cu") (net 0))
 (segment (start 148.082 82.296) (end 148.082 82.804) (width 0.25) (layer "F.Cu") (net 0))
 (segment (start 148.082 82.804) (end 146.886 84) (width 0.25) (layer "F.Cu") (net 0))
 (segment (start 146.886 84) (end 146 84) (width 0.25) (layer "F.Cu") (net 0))
 (segment (start 159.565 84) (end 160.655 85.09) (width 0.25) (layer "F.Cu") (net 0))
 (segment (start 160.655 85.09) (end 160.655 86.995) (width 0.25) (layer "F.Cu") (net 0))
 (segment (start 160.655 86.995) (end 163.83 90.17) (width 0.25) (layer "F.Cu") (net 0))
 (segment (start 159.335 82.5) (end 161.29 84.455) (width 0.25) (layer "F.Cu") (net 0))
 (segment (start 161.29 84.455) (end 161.29 85.09) (width 0.25) (layer "F.Cu") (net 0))
 (segment (start 161.29 85.09) (end 163.83 87.63) (width 0.25) (layer "F.Cu") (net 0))
 (segment (start 159.51 79.5) (end 162.56 82.55) (width 0.25) (layer "F.Cu") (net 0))
 (segment (start 162.56 82.55) (end 163.83 82.55) (width 0.25) (layer "F.Cu") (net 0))
 (segment (start 159.915 78) (end 161.925 80.01) (width 0.25) (layer "F.Cu") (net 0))
 (segment (start 161.925 80.01) (end 163.83 80.01) (width 0.25) (layer "F.Cu") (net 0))
 (segment (start 160.955 76.5) (end 161.925 77.47) (width 0.25) (layer "F.Cu") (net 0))
 (segment (start 161.925 77.47) (end 163.83 77.47) (width 0.25) (layer "F.Cu") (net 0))
 (segment (start 163.76 75) (end 163.83 74.93) (width 0.25) (layer "F.Cu") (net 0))
 (segment (start 145.235 84) (end 144.145 85.09) (width 0.25) (layer "F.Cu") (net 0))
 (segment (start 144.145 85.09) (end 144.145 86.995) (width 0.25) (layer "F.Cu") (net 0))
 (segment (start 144.145 86.995) (end 140.97 90.17) (width 0.25) (layer "F.Cu") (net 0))
 (segment (start 144.83 82.5) (end 143.51 83.82) (width 0.25) (layer "F.Cu") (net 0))
 (segment (start 143.51 83.82) (end 143.51 85.09) (width 0.25) (layer "F.Cu") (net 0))
 (segment (start 143.51 85.09) (end 140.97 87.63) (width 0.25) (layer "F.Cu") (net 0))
 (segment (start 145.06 81) (end 140.97 85.09) (width 0.25) (layer "F.Cu") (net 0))
 (segment (start 144.655 79.5) (end 141.605 82.55) (width 0.25) (layer "F.Cu") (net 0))
 (segment (start 141.605 82.55) (end 140.97 82.55) (width 0.25) (layer "F.Cu") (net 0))
 (segment (start 144.885 78) (end 142.875 80.01) (width 0.25) (layer "F.Cu") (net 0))
 (segment (start 142.875 80.01) (end 140.97 80.01) (width 0.25) (layer "F.Cu") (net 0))
 (segment (start 143.845 76.5) (end 142.875 77.47) (width 0.25) (layer "F.Cu") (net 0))
 (segment (start 142.875 77.47) (end 140.97 77.47) (width 0.25) (layer "F.Cu") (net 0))
 (segment (start 151.014 77.989) (end 151.765 78.74) (width 0.25) (layer "F.Cu") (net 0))
 (segment (start 151.765 78.74) (end 151.765 84.455) (width 0.25) (layer "F.Cu") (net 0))
 (segment (start 153.786 77.989) (end 153.035 78.74) (width 0.25) (layer "F.Cu") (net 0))
 (segment (start 153.035 78.74) (end 153.035 84.455) (width 0.25) (layer "F.Cu") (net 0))
 (segment (start 150.825 85.395) (end 151.765 84.455) (width 0.25) (layer "F.Cu") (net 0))
 (segment (start 153.975 85.395) (end 153.035 84.455) (width 0.25) (layer "F.Cu") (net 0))
 (segment (start 156.515 88.595) (end 156.845 88.265) (width 0.25) (layer "F.Cu") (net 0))
 (segment (start 156.845 88.265) (end 156.845 86.36) (width 0.25) (layer "F.Cu") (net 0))
 (segment (start 156.845 86.36) (end 157.705 85.5) (width 0.25) (layer "F.Cu") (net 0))
 (segment (start 157.705 85.5) (end 158.5 85.5) (width 0.25) (layer "F.Cu") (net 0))
 (segment (start 148.285 88.595) (end 147.955 88.265) (width 0.25) (layer "F.Cu") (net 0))
 (segment (start 147.955 88.265) (end 147.955 86.36) (width 0.25) (layer "F.Cu") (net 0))
 (segment (start 147.955 86.36) (end 147.095 85.5) (width 0.25) (layer "F.Cu") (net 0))
 (segment (start 147.095 85.5) (end 146 85.5) (width 0.25) (layer "F.Cu") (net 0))
 (segment (start 158.5 85.5) (end 157.636 85.5) (width 0.25) (layer "F.Cu") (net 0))
 (segment (start 146 82.5) (end 144.83 82.5) (width 0.25) (layer "F.Cu") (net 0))
 (segment (start 143.83 92.71) (end 144.145 92.395) (width 0.25) (layer "F.Cu") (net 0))
 (segment (start 146 87.68) (end 140.97 92.71) (width 0.25) (layer "F.Cu") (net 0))
 (segment (start 155.35 80.589) (end 158.089 80.589) (width 0.25) (layer "F.Cu") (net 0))
 (segment (start 158.5 79.5) (end 159.51 79.5) (width 0.25) (layer "F.Cu") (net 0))
 (segment (start 149.3425 91.525) (end 144.375 91.525) (width 0.25) (layer "F.Cu") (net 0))
 (segment (start 149.45 77.989) (end 151.014 77.989) (width 0.25) (layer "F.Cu") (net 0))
 (segment (start 146 76.5) (end 143.845 76.5) (width 0.25) (layer "F.Cu") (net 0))
 (segment (start 149.9 88.595) (end 148.285 88.595) (width 0.25) (layer "F.Cu") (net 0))
 (segment (start 155.35 77.989) (end 153.786 77.989) (width 0.25) (layer "F.Cu") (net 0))
 (segment (start 149.45 79.289) (end 147.869 79.289) (width 0.25) (layer "F.Cu") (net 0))
 (segment (start 158.5 87.38) (end 163.83 92.71) (width 0.25) (layer "F.Cu") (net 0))
 (segment (start 159.105 81) (end 163.195 85.09) (width 0.25) (layer "F.Cu") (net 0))
 (segment (start 144.375 91.525) (end 144.145 91.755) (width 0.25) (layer "F.Cu") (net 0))
 (segment (start 160.655 90.575) (end 156.337 90.575) (width 0.25) (layer "F.Cu") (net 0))
 (segment (start 149.45 81.889) (end 148.489 81.889) (width 0.25) (layer "F.Cu") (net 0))
 (segment (start 155.35 81.889) (end 156.311 81.889) (width 0.25) (layer "F.Cu") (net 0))
 (segment (start 158.5 76.5) (end 160.955 76.5) (width 0.25) (layer "F.Cu") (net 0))
 (segment (start 149.7925 91.075) (end 149.3425 91.525) (width 0.25) (layer "F.Cu") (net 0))
 (segment (start 155.837 91.075) (end 149.7925 91.075) (width 0.25) (layer "F.Cu") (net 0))
 (segment (start 158.5 78) (end 159.915 78) (width 0.25) (layer "F.Cu") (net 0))
 (segment (start 146 79.5) (end 144.655 79.5) (width 0.25) (layer "F.Cu") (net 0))
 (segment (start 156.337 93.575) (end 160.655 93.575) (width 0.25) (layer "F.Cu") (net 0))
 (segment (start 146 85.5) (end 146 87.68) (width 0.25) (layer "F.Cu") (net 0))
 (segment (start 146 84) (end 145.235 84) (width 0.25) (layer "F.Cu") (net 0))
 (segment (start 158.5 84) (end 159.565 84) (width 0.25) (layer "F.Cu") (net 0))
 (segment (start 149.45 80.589) (end 146.411 80.589) (width 0.25) (layer "F.Cu") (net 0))
 (segment (start 140.97 74.93) (end 147.066 74.93) (width 0.25) (layer "F.Cu") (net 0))
 (segment (start 149.2725 92.555) (end 149.7925 93.075) (width 0.25) (layer "F.Cu") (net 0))
 (segment (start 146 78) (end 144.885 78) (width 0.25) (layer "F.Cu") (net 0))
 (segment (start 158.5 75) (end 157.664 75) (width 0.25) (layer "F.Cu") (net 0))
 (segment (start 149.45 81.239) (end 147.869 81.239) (width 0.25) (layer "F.Cu") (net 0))
 (segment (start 156.337 90.575) (end 155.837 91.075) (width 0.25) (layer "F.Cu") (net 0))
 (segment (start 158.5 85.5) (end 158.5 87.38) (width 0.25) (layer "F.Cu") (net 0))
 (segment (start 140.97 92.71) (end 143.83 92.71) (width 0.25) (layer "F.Cu") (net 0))
 (segment (start 149.7925 93.075) (end 155.837 93.075) (width 0.25) (layer "F.Cu") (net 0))
 (segment (start 149.45 79.939) (end 146.439 79.939) (width 0.25) (layer "F.Cu") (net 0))
 (segment (start 155.35 81.239) (end 156.677 81.239) (width 0.25) (layer "F.Cu") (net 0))
 (segment (start 146 85.5) (end 146.91 85.5) (width 0.25) (layer "F.Cu") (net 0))
 (segment (start 158.5 82.5) (end 159.335 82.5) (width 0.25) (layer "F.Cu") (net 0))
 (segment (start 158.089 80.589) (end 158.5 81) (width 0.25) (layer "F.Cu") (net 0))
 (segment (start 155.35 79.939) (end 158.061 79.939) (width 0.25) (layer "F.Cu") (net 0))
 (segment (start 158.5 75) (end 163.76 75) (width 0.25) (layer "F.Cu") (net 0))
 (segment (start 163.195 85.09) (end 163.83 85.09) (width 0.25) (layer "F.Cu") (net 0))
 (segment (start 154.9 85.395) (end 153.975 85.395) (width 0.25) (layer "F.Cu") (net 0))
 (segment (start 149.9 85.395) (end 150.825 85.395) (width 0.25) (layer "F.Cu") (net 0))
 (segment (start 155.837 93.075) (end 156.337 93.575) (width 0.25) (layer "F.Cu") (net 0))
 (segment (start 154.9 88.595) (end 156.515 88.595) (width 0.25) (layer "F.Cu") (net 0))
 (segment (start 155.35 79.289) (end 156.677 79.289) (width 0.25) (layer "F.Cu") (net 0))
 (segment (start 144.145 92.395) (end 144.305 92.555) (width 0.25) (layer "F.Cu") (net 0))
 (segment (start 146 81) (end 145.06 81) (width 0.25) (layer "F.Cu") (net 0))
 (segment (start 155.35 78.639) (end 156.311 78.639) (width 0.25) (layer "F.Cu") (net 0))
 (segment (start 144.305 92.555) (end 149.2725 92.555) (width 0.25) (layer "F.Cu") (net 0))
 (segment (start 149.45 78.639) (end 148.437 78.639) (width 0.25) (layer "F.Cu") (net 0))
 (segment (start 162.56 76.2) (end 163.83 74.93) (width 0.25) (layer "B.Cu") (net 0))
 (segment (start 163.1 78.2) (end 163.83 77.47) (width 0.25) (layer "B.Cu") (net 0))
 (segment (start 163.64 80.2) (end 163.83 80.01) (width 0.25) (layer "B.Cu") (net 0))
 (segment (start 163.48 82.2) (end 163.83 82.55) (width 0.25) (layer "B.Cu") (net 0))
 (segment (start 162.94 84.2) (end 163.83 85.09) (width 0.25) (layer "B.Cu") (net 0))
 (segment (start 162.4 86.2) (end 163.83 87.63) (width 0.25) (layer "B.Cu") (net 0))
 (segment (start 142.24 76.2) (end 140.97 74.93) (width 0.25) (layer "B.Cu") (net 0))
 (segment (start 141.7 78.2) (end 140.97 77.47) (width 0.25) (layer "B.Cu") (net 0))
 (segment (start 141.16 80.2) (end 140.97 80.01) (width 0.25) (layer "B.Cu") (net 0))
 (segment (start 141.32 82.2) (end 140.97 82.55) (width 0.25) (layer "B.Cu") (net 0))
 (segment (start 141.86 84.2) (end 140.97 85.09) (width 0.25) (layer "B.Cu") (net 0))
 (segment (start 142.4 86.2) (end 140.97 87.63) (width 0.25) (layer "B.Cu") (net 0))
 (segment (start 161.86 88.2) (end 163.83 90.17) (width 0.25) (layer "B.Cu") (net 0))
 (segment (start 161.32 90.2) (end 163.83 92.71) (width 0.25) (layer "B.Cu") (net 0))
 (segment (start 142.94 88.2) (end 140.97 90.17) (width 0.25) (layer "B.Cu") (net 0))
 (segment (start 143.48 90.2) (end 140.97 92.71) (width 0.25) (layer "B.Cu") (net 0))
 (segment (start 147.195 80.01) (end 145.385 78.2) (width 0.25) (layer "B.Cu") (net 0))
 (segment (start 146.465 81.28) (end 145.385 80.2) (width 0.25) (layer "B.Cu") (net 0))
 (segment (start 145.735 82.55) (end 145.385 82.2) (width 0.25) (layer "B.Cu") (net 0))
 (segment (start 145.765 83.82) (end 145.385 84.2) (width 0.25) (layer "B.Cu") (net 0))
 (segment (start 146.495 85.09) (end 145.385 86.2) (width 0.25) (layer "B.Cu") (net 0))
 (segment (start 147.225 86.36) (end 145.385 88.2) (width 0.25) (layer "B.Cu") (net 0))
 (segment (start 147.75 87.835) (end 145.385 90.2) (width 0.25) (layer "B.Cu") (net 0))
 (segment (start 157.05 87.865) (end 159.385 90.2) (width 0.25) (layer "B.Cu") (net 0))
 (segment (start 157.545 86.36) (end 159.385 88.2) (width 0.25) (layer "B.Cu") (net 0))
 (segment (start 158.275 85.09) (end 159.385 86.2) (width 0.25) (layer "B.Cu") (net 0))
 (segment (start 159.005 83.82) (end 159.385 84.2) (width 0.25) (layer "B.Cu") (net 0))
 (segment (start 159.035 82.55) (end 159.385 82.2) (width 0.25) (layer "B.Cu") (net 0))
 (segment (start 158.305 81.28) (end 159.385 80.2) (width 0.25) (layer "B.Cu") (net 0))
 (segment (start 157.575 80.01) (end 159.385 78.2) (width 0.25) (layer "B.Cu") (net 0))
 (segment (start 157.05 78.535) (end 159.385 76.2) (width 0.25) (layer "B.Cu") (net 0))
 (segment (start 147.75 78.565) (end 145.385 76.2) (width 0.25) (layer "B.Cu") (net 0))
 (segment (start 157.05 85.09) (end 158.275 85.09) (width 0.25) (layer "B.Cu") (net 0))
 (segment (start 157.05 80.01) (end 157.575 80.01) (width 0.25) (layer "B.Cu") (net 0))
 (segment (start 159.385 86.2) (end 162.4 86.2) (width 0.25) (layer "B.Cu") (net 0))
 (segment (start 149.7 86.36) (end 147.75 86.36) (width 0.25) (layer "B.Cu") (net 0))
 (segment (start 145.385 90.2) (end 143.48 90.2) (width 0.25) (layer "B.Cu") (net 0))
 (segment (start 157.05 87.63) (end 157.05 87.865) (width 0.25) (layer "B.Cu") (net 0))
 (segment (start 147.75 80.01) (end 147.195 80.01) (width 0.25) (layer "B.Cu") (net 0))
 (segment (start 145.385 76.2) (end 142.24 76.2) (width 0.25) (layer "B.Cu") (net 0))
 (segment (start 147.75 81.28) (end 146.465 81.28) (width 0.25) (layer "B.Cu") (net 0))
 (segment (start 145.385 86.2) (end 142.4 86.2) (width 0.25) (layer "B.Cu") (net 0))
 (segment (start 145.385 80.2) (end 141.16 80.2) (width 0.25) (layer "B.Cu") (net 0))
 (segment (start 157.05 86.36) (end 157.545 86.36) (width 0.25) (layer "B.Cu") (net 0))
 (segment (start 149.7 82.55) (end 147.75 82.55) (width 0.25) (layer "B.Cu") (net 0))
 (segment (start 155.1 87.63) (end 157.05 87.63) (width 0.25) (layer "B.Cu") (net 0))
 (segment (start 145.385 82.2) (end 141.32 82.2) (width 0.25) (layer "B.Cu") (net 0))
 (segment (start 155.1 82.55) (end 157.05 82.55) (width 0.25) (layer "B.Cu") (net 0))
 (segment (start 149.7 83.82) (end 147.75 83.82) (width 0.25) (layer "B.Cu") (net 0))
 (segment (start 159.385 84.2) (end 162.94 84.2) (width 0.25) (layer "B.Cu") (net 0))
 (segment (start 145.385 78.2) (end 141.7 78.2) (width 0.25) (layer "B.Cu") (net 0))
 (segment (start 155.1 78.74) (end 157.05 78.74) (width 0.25) (layer "B.Cu") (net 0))
 (segment (start 159.385 78.2) (end 163.1 78.2) (width 0.25) (layer "B.Cu") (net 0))
 (segment (start 159.385 80.2) (end 163.64 80.2) (width 0.25) (layer "B.Cu") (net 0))
 (segment (start 149.7 85.09) (end 147.75 85.09) (width 0.25) (layer "B.Cu") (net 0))
 (segment (start 147.75 82.55) (end 145.735 82.55) (width 0.25) (layer "B.Cu") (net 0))
 (segment (start 147.75 86.36) (end 147.225 86.36) (width 0.25) (layer "B.Cu") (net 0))
 (segment (start 157.05 78.74) (end 157.05 78.535) (width 0.25) (layer "B.Cu") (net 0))
 (segment (start 147.75 85.09) (end 146.495 85.09) (width 0.25) (layer "B.Cu") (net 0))
 (segment (start 155.1 80.01) (end 157.05 80.01) (width 0.25) (layer "B.Cu") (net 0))
 (segment (start 159.385 76.2) (end 162.56 76.2) (width 0.25) (layer "B.Cu") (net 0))
 (segment (start 147.75 78.74) (end 147.75 78.565) (width 0.25) (layer "B.Cu") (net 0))
 (segment (start 155.1 85.09) (end 157.05 85.09) (width 0.25) (layer "B.Cu") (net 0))
 (segment (start 145.385 84.2) (end 141.86 84.2) (width 0.25) (layer "B.Cu") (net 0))
 (segment (start 155.1 86.36) (end 157.05 86.36) (width 0.25) (layer "B.Cu") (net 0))
 (segment (start 149.7 87.63) (end 147.75 87.63) (width 0.25) (layer "B.Cu") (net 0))
 (segment (start 159.385 90.2) (end 161.32 90.2) (width 0.25) (layer "B.Cu") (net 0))
 (segment (start 147.75 87.63) (end 147.75 87.835) (width 0.25) (layer "B.Cu") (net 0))
 (segment (start 147.75 83.82) (end 145.765 83.82) (width 0.25) (layer "B.Cu") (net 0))
 (segment (start 159.385 88.2) (end 161.86 88.2) (width 0.25) (layer "B.Cu") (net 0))
 (segment (start 157.05 83.82) (end 159.005 83.82) (width 0.25) (layer "B.Cu") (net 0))
 (segment (start 155.1 83.82) (end 157.05 83.82) (width 0.25) (layer "B.Cu") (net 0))
 (segment (start 155.1 81.28) (end 157.05 81.28) (width 0.25) (layer "B.Cu") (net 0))
 (segment (start 157.05 81.28) (end 158.305 81.28) (width 0.25) (layer "B.Cu") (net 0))
 (segment (start 157.05 82.55) (end 159.035 82.55) (width 0.25) (layer "B.Cu") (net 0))
 (segment (start 159.385 82.2) (end 163.48 82.2) (width 0.25) (layer "B.Cu") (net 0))
 (segment (start 145.385 88.2) (end 142.94 88.2) (width 0.25) (layer "B.Cu") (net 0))
 (segment (start 149.7 80.01) (end 147.75 80.01) (width 0.25) (layer "B.Cu") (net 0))
 (segment (start 149.7 81.28) (end 147.75 81.28) (width 0.25) (layer "B.Cu") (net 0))
 (segment (start 149.7 78.74) (end 147.75 78.74) (width 0.25) (layer "B.Cu") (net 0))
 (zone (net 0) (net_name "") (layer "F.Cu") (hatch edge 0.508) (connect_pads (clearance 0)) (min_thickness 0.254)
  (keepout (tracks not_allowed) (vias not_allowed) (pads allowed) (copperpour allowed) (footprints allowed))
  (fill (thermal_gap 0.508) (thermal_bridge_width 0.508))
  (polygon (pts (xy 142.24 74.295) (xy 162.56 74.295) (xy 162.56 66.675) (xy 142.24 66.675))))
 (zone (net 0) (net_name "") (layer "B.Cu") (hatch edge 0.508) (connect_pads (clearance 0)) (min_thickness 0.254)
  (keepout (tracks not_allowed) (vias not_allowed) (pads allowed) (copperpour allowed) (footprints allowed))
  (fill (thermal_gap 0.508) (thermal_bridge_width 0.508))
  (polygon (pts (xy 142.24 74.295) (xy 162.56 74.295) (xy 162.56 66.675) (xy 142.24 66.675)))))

